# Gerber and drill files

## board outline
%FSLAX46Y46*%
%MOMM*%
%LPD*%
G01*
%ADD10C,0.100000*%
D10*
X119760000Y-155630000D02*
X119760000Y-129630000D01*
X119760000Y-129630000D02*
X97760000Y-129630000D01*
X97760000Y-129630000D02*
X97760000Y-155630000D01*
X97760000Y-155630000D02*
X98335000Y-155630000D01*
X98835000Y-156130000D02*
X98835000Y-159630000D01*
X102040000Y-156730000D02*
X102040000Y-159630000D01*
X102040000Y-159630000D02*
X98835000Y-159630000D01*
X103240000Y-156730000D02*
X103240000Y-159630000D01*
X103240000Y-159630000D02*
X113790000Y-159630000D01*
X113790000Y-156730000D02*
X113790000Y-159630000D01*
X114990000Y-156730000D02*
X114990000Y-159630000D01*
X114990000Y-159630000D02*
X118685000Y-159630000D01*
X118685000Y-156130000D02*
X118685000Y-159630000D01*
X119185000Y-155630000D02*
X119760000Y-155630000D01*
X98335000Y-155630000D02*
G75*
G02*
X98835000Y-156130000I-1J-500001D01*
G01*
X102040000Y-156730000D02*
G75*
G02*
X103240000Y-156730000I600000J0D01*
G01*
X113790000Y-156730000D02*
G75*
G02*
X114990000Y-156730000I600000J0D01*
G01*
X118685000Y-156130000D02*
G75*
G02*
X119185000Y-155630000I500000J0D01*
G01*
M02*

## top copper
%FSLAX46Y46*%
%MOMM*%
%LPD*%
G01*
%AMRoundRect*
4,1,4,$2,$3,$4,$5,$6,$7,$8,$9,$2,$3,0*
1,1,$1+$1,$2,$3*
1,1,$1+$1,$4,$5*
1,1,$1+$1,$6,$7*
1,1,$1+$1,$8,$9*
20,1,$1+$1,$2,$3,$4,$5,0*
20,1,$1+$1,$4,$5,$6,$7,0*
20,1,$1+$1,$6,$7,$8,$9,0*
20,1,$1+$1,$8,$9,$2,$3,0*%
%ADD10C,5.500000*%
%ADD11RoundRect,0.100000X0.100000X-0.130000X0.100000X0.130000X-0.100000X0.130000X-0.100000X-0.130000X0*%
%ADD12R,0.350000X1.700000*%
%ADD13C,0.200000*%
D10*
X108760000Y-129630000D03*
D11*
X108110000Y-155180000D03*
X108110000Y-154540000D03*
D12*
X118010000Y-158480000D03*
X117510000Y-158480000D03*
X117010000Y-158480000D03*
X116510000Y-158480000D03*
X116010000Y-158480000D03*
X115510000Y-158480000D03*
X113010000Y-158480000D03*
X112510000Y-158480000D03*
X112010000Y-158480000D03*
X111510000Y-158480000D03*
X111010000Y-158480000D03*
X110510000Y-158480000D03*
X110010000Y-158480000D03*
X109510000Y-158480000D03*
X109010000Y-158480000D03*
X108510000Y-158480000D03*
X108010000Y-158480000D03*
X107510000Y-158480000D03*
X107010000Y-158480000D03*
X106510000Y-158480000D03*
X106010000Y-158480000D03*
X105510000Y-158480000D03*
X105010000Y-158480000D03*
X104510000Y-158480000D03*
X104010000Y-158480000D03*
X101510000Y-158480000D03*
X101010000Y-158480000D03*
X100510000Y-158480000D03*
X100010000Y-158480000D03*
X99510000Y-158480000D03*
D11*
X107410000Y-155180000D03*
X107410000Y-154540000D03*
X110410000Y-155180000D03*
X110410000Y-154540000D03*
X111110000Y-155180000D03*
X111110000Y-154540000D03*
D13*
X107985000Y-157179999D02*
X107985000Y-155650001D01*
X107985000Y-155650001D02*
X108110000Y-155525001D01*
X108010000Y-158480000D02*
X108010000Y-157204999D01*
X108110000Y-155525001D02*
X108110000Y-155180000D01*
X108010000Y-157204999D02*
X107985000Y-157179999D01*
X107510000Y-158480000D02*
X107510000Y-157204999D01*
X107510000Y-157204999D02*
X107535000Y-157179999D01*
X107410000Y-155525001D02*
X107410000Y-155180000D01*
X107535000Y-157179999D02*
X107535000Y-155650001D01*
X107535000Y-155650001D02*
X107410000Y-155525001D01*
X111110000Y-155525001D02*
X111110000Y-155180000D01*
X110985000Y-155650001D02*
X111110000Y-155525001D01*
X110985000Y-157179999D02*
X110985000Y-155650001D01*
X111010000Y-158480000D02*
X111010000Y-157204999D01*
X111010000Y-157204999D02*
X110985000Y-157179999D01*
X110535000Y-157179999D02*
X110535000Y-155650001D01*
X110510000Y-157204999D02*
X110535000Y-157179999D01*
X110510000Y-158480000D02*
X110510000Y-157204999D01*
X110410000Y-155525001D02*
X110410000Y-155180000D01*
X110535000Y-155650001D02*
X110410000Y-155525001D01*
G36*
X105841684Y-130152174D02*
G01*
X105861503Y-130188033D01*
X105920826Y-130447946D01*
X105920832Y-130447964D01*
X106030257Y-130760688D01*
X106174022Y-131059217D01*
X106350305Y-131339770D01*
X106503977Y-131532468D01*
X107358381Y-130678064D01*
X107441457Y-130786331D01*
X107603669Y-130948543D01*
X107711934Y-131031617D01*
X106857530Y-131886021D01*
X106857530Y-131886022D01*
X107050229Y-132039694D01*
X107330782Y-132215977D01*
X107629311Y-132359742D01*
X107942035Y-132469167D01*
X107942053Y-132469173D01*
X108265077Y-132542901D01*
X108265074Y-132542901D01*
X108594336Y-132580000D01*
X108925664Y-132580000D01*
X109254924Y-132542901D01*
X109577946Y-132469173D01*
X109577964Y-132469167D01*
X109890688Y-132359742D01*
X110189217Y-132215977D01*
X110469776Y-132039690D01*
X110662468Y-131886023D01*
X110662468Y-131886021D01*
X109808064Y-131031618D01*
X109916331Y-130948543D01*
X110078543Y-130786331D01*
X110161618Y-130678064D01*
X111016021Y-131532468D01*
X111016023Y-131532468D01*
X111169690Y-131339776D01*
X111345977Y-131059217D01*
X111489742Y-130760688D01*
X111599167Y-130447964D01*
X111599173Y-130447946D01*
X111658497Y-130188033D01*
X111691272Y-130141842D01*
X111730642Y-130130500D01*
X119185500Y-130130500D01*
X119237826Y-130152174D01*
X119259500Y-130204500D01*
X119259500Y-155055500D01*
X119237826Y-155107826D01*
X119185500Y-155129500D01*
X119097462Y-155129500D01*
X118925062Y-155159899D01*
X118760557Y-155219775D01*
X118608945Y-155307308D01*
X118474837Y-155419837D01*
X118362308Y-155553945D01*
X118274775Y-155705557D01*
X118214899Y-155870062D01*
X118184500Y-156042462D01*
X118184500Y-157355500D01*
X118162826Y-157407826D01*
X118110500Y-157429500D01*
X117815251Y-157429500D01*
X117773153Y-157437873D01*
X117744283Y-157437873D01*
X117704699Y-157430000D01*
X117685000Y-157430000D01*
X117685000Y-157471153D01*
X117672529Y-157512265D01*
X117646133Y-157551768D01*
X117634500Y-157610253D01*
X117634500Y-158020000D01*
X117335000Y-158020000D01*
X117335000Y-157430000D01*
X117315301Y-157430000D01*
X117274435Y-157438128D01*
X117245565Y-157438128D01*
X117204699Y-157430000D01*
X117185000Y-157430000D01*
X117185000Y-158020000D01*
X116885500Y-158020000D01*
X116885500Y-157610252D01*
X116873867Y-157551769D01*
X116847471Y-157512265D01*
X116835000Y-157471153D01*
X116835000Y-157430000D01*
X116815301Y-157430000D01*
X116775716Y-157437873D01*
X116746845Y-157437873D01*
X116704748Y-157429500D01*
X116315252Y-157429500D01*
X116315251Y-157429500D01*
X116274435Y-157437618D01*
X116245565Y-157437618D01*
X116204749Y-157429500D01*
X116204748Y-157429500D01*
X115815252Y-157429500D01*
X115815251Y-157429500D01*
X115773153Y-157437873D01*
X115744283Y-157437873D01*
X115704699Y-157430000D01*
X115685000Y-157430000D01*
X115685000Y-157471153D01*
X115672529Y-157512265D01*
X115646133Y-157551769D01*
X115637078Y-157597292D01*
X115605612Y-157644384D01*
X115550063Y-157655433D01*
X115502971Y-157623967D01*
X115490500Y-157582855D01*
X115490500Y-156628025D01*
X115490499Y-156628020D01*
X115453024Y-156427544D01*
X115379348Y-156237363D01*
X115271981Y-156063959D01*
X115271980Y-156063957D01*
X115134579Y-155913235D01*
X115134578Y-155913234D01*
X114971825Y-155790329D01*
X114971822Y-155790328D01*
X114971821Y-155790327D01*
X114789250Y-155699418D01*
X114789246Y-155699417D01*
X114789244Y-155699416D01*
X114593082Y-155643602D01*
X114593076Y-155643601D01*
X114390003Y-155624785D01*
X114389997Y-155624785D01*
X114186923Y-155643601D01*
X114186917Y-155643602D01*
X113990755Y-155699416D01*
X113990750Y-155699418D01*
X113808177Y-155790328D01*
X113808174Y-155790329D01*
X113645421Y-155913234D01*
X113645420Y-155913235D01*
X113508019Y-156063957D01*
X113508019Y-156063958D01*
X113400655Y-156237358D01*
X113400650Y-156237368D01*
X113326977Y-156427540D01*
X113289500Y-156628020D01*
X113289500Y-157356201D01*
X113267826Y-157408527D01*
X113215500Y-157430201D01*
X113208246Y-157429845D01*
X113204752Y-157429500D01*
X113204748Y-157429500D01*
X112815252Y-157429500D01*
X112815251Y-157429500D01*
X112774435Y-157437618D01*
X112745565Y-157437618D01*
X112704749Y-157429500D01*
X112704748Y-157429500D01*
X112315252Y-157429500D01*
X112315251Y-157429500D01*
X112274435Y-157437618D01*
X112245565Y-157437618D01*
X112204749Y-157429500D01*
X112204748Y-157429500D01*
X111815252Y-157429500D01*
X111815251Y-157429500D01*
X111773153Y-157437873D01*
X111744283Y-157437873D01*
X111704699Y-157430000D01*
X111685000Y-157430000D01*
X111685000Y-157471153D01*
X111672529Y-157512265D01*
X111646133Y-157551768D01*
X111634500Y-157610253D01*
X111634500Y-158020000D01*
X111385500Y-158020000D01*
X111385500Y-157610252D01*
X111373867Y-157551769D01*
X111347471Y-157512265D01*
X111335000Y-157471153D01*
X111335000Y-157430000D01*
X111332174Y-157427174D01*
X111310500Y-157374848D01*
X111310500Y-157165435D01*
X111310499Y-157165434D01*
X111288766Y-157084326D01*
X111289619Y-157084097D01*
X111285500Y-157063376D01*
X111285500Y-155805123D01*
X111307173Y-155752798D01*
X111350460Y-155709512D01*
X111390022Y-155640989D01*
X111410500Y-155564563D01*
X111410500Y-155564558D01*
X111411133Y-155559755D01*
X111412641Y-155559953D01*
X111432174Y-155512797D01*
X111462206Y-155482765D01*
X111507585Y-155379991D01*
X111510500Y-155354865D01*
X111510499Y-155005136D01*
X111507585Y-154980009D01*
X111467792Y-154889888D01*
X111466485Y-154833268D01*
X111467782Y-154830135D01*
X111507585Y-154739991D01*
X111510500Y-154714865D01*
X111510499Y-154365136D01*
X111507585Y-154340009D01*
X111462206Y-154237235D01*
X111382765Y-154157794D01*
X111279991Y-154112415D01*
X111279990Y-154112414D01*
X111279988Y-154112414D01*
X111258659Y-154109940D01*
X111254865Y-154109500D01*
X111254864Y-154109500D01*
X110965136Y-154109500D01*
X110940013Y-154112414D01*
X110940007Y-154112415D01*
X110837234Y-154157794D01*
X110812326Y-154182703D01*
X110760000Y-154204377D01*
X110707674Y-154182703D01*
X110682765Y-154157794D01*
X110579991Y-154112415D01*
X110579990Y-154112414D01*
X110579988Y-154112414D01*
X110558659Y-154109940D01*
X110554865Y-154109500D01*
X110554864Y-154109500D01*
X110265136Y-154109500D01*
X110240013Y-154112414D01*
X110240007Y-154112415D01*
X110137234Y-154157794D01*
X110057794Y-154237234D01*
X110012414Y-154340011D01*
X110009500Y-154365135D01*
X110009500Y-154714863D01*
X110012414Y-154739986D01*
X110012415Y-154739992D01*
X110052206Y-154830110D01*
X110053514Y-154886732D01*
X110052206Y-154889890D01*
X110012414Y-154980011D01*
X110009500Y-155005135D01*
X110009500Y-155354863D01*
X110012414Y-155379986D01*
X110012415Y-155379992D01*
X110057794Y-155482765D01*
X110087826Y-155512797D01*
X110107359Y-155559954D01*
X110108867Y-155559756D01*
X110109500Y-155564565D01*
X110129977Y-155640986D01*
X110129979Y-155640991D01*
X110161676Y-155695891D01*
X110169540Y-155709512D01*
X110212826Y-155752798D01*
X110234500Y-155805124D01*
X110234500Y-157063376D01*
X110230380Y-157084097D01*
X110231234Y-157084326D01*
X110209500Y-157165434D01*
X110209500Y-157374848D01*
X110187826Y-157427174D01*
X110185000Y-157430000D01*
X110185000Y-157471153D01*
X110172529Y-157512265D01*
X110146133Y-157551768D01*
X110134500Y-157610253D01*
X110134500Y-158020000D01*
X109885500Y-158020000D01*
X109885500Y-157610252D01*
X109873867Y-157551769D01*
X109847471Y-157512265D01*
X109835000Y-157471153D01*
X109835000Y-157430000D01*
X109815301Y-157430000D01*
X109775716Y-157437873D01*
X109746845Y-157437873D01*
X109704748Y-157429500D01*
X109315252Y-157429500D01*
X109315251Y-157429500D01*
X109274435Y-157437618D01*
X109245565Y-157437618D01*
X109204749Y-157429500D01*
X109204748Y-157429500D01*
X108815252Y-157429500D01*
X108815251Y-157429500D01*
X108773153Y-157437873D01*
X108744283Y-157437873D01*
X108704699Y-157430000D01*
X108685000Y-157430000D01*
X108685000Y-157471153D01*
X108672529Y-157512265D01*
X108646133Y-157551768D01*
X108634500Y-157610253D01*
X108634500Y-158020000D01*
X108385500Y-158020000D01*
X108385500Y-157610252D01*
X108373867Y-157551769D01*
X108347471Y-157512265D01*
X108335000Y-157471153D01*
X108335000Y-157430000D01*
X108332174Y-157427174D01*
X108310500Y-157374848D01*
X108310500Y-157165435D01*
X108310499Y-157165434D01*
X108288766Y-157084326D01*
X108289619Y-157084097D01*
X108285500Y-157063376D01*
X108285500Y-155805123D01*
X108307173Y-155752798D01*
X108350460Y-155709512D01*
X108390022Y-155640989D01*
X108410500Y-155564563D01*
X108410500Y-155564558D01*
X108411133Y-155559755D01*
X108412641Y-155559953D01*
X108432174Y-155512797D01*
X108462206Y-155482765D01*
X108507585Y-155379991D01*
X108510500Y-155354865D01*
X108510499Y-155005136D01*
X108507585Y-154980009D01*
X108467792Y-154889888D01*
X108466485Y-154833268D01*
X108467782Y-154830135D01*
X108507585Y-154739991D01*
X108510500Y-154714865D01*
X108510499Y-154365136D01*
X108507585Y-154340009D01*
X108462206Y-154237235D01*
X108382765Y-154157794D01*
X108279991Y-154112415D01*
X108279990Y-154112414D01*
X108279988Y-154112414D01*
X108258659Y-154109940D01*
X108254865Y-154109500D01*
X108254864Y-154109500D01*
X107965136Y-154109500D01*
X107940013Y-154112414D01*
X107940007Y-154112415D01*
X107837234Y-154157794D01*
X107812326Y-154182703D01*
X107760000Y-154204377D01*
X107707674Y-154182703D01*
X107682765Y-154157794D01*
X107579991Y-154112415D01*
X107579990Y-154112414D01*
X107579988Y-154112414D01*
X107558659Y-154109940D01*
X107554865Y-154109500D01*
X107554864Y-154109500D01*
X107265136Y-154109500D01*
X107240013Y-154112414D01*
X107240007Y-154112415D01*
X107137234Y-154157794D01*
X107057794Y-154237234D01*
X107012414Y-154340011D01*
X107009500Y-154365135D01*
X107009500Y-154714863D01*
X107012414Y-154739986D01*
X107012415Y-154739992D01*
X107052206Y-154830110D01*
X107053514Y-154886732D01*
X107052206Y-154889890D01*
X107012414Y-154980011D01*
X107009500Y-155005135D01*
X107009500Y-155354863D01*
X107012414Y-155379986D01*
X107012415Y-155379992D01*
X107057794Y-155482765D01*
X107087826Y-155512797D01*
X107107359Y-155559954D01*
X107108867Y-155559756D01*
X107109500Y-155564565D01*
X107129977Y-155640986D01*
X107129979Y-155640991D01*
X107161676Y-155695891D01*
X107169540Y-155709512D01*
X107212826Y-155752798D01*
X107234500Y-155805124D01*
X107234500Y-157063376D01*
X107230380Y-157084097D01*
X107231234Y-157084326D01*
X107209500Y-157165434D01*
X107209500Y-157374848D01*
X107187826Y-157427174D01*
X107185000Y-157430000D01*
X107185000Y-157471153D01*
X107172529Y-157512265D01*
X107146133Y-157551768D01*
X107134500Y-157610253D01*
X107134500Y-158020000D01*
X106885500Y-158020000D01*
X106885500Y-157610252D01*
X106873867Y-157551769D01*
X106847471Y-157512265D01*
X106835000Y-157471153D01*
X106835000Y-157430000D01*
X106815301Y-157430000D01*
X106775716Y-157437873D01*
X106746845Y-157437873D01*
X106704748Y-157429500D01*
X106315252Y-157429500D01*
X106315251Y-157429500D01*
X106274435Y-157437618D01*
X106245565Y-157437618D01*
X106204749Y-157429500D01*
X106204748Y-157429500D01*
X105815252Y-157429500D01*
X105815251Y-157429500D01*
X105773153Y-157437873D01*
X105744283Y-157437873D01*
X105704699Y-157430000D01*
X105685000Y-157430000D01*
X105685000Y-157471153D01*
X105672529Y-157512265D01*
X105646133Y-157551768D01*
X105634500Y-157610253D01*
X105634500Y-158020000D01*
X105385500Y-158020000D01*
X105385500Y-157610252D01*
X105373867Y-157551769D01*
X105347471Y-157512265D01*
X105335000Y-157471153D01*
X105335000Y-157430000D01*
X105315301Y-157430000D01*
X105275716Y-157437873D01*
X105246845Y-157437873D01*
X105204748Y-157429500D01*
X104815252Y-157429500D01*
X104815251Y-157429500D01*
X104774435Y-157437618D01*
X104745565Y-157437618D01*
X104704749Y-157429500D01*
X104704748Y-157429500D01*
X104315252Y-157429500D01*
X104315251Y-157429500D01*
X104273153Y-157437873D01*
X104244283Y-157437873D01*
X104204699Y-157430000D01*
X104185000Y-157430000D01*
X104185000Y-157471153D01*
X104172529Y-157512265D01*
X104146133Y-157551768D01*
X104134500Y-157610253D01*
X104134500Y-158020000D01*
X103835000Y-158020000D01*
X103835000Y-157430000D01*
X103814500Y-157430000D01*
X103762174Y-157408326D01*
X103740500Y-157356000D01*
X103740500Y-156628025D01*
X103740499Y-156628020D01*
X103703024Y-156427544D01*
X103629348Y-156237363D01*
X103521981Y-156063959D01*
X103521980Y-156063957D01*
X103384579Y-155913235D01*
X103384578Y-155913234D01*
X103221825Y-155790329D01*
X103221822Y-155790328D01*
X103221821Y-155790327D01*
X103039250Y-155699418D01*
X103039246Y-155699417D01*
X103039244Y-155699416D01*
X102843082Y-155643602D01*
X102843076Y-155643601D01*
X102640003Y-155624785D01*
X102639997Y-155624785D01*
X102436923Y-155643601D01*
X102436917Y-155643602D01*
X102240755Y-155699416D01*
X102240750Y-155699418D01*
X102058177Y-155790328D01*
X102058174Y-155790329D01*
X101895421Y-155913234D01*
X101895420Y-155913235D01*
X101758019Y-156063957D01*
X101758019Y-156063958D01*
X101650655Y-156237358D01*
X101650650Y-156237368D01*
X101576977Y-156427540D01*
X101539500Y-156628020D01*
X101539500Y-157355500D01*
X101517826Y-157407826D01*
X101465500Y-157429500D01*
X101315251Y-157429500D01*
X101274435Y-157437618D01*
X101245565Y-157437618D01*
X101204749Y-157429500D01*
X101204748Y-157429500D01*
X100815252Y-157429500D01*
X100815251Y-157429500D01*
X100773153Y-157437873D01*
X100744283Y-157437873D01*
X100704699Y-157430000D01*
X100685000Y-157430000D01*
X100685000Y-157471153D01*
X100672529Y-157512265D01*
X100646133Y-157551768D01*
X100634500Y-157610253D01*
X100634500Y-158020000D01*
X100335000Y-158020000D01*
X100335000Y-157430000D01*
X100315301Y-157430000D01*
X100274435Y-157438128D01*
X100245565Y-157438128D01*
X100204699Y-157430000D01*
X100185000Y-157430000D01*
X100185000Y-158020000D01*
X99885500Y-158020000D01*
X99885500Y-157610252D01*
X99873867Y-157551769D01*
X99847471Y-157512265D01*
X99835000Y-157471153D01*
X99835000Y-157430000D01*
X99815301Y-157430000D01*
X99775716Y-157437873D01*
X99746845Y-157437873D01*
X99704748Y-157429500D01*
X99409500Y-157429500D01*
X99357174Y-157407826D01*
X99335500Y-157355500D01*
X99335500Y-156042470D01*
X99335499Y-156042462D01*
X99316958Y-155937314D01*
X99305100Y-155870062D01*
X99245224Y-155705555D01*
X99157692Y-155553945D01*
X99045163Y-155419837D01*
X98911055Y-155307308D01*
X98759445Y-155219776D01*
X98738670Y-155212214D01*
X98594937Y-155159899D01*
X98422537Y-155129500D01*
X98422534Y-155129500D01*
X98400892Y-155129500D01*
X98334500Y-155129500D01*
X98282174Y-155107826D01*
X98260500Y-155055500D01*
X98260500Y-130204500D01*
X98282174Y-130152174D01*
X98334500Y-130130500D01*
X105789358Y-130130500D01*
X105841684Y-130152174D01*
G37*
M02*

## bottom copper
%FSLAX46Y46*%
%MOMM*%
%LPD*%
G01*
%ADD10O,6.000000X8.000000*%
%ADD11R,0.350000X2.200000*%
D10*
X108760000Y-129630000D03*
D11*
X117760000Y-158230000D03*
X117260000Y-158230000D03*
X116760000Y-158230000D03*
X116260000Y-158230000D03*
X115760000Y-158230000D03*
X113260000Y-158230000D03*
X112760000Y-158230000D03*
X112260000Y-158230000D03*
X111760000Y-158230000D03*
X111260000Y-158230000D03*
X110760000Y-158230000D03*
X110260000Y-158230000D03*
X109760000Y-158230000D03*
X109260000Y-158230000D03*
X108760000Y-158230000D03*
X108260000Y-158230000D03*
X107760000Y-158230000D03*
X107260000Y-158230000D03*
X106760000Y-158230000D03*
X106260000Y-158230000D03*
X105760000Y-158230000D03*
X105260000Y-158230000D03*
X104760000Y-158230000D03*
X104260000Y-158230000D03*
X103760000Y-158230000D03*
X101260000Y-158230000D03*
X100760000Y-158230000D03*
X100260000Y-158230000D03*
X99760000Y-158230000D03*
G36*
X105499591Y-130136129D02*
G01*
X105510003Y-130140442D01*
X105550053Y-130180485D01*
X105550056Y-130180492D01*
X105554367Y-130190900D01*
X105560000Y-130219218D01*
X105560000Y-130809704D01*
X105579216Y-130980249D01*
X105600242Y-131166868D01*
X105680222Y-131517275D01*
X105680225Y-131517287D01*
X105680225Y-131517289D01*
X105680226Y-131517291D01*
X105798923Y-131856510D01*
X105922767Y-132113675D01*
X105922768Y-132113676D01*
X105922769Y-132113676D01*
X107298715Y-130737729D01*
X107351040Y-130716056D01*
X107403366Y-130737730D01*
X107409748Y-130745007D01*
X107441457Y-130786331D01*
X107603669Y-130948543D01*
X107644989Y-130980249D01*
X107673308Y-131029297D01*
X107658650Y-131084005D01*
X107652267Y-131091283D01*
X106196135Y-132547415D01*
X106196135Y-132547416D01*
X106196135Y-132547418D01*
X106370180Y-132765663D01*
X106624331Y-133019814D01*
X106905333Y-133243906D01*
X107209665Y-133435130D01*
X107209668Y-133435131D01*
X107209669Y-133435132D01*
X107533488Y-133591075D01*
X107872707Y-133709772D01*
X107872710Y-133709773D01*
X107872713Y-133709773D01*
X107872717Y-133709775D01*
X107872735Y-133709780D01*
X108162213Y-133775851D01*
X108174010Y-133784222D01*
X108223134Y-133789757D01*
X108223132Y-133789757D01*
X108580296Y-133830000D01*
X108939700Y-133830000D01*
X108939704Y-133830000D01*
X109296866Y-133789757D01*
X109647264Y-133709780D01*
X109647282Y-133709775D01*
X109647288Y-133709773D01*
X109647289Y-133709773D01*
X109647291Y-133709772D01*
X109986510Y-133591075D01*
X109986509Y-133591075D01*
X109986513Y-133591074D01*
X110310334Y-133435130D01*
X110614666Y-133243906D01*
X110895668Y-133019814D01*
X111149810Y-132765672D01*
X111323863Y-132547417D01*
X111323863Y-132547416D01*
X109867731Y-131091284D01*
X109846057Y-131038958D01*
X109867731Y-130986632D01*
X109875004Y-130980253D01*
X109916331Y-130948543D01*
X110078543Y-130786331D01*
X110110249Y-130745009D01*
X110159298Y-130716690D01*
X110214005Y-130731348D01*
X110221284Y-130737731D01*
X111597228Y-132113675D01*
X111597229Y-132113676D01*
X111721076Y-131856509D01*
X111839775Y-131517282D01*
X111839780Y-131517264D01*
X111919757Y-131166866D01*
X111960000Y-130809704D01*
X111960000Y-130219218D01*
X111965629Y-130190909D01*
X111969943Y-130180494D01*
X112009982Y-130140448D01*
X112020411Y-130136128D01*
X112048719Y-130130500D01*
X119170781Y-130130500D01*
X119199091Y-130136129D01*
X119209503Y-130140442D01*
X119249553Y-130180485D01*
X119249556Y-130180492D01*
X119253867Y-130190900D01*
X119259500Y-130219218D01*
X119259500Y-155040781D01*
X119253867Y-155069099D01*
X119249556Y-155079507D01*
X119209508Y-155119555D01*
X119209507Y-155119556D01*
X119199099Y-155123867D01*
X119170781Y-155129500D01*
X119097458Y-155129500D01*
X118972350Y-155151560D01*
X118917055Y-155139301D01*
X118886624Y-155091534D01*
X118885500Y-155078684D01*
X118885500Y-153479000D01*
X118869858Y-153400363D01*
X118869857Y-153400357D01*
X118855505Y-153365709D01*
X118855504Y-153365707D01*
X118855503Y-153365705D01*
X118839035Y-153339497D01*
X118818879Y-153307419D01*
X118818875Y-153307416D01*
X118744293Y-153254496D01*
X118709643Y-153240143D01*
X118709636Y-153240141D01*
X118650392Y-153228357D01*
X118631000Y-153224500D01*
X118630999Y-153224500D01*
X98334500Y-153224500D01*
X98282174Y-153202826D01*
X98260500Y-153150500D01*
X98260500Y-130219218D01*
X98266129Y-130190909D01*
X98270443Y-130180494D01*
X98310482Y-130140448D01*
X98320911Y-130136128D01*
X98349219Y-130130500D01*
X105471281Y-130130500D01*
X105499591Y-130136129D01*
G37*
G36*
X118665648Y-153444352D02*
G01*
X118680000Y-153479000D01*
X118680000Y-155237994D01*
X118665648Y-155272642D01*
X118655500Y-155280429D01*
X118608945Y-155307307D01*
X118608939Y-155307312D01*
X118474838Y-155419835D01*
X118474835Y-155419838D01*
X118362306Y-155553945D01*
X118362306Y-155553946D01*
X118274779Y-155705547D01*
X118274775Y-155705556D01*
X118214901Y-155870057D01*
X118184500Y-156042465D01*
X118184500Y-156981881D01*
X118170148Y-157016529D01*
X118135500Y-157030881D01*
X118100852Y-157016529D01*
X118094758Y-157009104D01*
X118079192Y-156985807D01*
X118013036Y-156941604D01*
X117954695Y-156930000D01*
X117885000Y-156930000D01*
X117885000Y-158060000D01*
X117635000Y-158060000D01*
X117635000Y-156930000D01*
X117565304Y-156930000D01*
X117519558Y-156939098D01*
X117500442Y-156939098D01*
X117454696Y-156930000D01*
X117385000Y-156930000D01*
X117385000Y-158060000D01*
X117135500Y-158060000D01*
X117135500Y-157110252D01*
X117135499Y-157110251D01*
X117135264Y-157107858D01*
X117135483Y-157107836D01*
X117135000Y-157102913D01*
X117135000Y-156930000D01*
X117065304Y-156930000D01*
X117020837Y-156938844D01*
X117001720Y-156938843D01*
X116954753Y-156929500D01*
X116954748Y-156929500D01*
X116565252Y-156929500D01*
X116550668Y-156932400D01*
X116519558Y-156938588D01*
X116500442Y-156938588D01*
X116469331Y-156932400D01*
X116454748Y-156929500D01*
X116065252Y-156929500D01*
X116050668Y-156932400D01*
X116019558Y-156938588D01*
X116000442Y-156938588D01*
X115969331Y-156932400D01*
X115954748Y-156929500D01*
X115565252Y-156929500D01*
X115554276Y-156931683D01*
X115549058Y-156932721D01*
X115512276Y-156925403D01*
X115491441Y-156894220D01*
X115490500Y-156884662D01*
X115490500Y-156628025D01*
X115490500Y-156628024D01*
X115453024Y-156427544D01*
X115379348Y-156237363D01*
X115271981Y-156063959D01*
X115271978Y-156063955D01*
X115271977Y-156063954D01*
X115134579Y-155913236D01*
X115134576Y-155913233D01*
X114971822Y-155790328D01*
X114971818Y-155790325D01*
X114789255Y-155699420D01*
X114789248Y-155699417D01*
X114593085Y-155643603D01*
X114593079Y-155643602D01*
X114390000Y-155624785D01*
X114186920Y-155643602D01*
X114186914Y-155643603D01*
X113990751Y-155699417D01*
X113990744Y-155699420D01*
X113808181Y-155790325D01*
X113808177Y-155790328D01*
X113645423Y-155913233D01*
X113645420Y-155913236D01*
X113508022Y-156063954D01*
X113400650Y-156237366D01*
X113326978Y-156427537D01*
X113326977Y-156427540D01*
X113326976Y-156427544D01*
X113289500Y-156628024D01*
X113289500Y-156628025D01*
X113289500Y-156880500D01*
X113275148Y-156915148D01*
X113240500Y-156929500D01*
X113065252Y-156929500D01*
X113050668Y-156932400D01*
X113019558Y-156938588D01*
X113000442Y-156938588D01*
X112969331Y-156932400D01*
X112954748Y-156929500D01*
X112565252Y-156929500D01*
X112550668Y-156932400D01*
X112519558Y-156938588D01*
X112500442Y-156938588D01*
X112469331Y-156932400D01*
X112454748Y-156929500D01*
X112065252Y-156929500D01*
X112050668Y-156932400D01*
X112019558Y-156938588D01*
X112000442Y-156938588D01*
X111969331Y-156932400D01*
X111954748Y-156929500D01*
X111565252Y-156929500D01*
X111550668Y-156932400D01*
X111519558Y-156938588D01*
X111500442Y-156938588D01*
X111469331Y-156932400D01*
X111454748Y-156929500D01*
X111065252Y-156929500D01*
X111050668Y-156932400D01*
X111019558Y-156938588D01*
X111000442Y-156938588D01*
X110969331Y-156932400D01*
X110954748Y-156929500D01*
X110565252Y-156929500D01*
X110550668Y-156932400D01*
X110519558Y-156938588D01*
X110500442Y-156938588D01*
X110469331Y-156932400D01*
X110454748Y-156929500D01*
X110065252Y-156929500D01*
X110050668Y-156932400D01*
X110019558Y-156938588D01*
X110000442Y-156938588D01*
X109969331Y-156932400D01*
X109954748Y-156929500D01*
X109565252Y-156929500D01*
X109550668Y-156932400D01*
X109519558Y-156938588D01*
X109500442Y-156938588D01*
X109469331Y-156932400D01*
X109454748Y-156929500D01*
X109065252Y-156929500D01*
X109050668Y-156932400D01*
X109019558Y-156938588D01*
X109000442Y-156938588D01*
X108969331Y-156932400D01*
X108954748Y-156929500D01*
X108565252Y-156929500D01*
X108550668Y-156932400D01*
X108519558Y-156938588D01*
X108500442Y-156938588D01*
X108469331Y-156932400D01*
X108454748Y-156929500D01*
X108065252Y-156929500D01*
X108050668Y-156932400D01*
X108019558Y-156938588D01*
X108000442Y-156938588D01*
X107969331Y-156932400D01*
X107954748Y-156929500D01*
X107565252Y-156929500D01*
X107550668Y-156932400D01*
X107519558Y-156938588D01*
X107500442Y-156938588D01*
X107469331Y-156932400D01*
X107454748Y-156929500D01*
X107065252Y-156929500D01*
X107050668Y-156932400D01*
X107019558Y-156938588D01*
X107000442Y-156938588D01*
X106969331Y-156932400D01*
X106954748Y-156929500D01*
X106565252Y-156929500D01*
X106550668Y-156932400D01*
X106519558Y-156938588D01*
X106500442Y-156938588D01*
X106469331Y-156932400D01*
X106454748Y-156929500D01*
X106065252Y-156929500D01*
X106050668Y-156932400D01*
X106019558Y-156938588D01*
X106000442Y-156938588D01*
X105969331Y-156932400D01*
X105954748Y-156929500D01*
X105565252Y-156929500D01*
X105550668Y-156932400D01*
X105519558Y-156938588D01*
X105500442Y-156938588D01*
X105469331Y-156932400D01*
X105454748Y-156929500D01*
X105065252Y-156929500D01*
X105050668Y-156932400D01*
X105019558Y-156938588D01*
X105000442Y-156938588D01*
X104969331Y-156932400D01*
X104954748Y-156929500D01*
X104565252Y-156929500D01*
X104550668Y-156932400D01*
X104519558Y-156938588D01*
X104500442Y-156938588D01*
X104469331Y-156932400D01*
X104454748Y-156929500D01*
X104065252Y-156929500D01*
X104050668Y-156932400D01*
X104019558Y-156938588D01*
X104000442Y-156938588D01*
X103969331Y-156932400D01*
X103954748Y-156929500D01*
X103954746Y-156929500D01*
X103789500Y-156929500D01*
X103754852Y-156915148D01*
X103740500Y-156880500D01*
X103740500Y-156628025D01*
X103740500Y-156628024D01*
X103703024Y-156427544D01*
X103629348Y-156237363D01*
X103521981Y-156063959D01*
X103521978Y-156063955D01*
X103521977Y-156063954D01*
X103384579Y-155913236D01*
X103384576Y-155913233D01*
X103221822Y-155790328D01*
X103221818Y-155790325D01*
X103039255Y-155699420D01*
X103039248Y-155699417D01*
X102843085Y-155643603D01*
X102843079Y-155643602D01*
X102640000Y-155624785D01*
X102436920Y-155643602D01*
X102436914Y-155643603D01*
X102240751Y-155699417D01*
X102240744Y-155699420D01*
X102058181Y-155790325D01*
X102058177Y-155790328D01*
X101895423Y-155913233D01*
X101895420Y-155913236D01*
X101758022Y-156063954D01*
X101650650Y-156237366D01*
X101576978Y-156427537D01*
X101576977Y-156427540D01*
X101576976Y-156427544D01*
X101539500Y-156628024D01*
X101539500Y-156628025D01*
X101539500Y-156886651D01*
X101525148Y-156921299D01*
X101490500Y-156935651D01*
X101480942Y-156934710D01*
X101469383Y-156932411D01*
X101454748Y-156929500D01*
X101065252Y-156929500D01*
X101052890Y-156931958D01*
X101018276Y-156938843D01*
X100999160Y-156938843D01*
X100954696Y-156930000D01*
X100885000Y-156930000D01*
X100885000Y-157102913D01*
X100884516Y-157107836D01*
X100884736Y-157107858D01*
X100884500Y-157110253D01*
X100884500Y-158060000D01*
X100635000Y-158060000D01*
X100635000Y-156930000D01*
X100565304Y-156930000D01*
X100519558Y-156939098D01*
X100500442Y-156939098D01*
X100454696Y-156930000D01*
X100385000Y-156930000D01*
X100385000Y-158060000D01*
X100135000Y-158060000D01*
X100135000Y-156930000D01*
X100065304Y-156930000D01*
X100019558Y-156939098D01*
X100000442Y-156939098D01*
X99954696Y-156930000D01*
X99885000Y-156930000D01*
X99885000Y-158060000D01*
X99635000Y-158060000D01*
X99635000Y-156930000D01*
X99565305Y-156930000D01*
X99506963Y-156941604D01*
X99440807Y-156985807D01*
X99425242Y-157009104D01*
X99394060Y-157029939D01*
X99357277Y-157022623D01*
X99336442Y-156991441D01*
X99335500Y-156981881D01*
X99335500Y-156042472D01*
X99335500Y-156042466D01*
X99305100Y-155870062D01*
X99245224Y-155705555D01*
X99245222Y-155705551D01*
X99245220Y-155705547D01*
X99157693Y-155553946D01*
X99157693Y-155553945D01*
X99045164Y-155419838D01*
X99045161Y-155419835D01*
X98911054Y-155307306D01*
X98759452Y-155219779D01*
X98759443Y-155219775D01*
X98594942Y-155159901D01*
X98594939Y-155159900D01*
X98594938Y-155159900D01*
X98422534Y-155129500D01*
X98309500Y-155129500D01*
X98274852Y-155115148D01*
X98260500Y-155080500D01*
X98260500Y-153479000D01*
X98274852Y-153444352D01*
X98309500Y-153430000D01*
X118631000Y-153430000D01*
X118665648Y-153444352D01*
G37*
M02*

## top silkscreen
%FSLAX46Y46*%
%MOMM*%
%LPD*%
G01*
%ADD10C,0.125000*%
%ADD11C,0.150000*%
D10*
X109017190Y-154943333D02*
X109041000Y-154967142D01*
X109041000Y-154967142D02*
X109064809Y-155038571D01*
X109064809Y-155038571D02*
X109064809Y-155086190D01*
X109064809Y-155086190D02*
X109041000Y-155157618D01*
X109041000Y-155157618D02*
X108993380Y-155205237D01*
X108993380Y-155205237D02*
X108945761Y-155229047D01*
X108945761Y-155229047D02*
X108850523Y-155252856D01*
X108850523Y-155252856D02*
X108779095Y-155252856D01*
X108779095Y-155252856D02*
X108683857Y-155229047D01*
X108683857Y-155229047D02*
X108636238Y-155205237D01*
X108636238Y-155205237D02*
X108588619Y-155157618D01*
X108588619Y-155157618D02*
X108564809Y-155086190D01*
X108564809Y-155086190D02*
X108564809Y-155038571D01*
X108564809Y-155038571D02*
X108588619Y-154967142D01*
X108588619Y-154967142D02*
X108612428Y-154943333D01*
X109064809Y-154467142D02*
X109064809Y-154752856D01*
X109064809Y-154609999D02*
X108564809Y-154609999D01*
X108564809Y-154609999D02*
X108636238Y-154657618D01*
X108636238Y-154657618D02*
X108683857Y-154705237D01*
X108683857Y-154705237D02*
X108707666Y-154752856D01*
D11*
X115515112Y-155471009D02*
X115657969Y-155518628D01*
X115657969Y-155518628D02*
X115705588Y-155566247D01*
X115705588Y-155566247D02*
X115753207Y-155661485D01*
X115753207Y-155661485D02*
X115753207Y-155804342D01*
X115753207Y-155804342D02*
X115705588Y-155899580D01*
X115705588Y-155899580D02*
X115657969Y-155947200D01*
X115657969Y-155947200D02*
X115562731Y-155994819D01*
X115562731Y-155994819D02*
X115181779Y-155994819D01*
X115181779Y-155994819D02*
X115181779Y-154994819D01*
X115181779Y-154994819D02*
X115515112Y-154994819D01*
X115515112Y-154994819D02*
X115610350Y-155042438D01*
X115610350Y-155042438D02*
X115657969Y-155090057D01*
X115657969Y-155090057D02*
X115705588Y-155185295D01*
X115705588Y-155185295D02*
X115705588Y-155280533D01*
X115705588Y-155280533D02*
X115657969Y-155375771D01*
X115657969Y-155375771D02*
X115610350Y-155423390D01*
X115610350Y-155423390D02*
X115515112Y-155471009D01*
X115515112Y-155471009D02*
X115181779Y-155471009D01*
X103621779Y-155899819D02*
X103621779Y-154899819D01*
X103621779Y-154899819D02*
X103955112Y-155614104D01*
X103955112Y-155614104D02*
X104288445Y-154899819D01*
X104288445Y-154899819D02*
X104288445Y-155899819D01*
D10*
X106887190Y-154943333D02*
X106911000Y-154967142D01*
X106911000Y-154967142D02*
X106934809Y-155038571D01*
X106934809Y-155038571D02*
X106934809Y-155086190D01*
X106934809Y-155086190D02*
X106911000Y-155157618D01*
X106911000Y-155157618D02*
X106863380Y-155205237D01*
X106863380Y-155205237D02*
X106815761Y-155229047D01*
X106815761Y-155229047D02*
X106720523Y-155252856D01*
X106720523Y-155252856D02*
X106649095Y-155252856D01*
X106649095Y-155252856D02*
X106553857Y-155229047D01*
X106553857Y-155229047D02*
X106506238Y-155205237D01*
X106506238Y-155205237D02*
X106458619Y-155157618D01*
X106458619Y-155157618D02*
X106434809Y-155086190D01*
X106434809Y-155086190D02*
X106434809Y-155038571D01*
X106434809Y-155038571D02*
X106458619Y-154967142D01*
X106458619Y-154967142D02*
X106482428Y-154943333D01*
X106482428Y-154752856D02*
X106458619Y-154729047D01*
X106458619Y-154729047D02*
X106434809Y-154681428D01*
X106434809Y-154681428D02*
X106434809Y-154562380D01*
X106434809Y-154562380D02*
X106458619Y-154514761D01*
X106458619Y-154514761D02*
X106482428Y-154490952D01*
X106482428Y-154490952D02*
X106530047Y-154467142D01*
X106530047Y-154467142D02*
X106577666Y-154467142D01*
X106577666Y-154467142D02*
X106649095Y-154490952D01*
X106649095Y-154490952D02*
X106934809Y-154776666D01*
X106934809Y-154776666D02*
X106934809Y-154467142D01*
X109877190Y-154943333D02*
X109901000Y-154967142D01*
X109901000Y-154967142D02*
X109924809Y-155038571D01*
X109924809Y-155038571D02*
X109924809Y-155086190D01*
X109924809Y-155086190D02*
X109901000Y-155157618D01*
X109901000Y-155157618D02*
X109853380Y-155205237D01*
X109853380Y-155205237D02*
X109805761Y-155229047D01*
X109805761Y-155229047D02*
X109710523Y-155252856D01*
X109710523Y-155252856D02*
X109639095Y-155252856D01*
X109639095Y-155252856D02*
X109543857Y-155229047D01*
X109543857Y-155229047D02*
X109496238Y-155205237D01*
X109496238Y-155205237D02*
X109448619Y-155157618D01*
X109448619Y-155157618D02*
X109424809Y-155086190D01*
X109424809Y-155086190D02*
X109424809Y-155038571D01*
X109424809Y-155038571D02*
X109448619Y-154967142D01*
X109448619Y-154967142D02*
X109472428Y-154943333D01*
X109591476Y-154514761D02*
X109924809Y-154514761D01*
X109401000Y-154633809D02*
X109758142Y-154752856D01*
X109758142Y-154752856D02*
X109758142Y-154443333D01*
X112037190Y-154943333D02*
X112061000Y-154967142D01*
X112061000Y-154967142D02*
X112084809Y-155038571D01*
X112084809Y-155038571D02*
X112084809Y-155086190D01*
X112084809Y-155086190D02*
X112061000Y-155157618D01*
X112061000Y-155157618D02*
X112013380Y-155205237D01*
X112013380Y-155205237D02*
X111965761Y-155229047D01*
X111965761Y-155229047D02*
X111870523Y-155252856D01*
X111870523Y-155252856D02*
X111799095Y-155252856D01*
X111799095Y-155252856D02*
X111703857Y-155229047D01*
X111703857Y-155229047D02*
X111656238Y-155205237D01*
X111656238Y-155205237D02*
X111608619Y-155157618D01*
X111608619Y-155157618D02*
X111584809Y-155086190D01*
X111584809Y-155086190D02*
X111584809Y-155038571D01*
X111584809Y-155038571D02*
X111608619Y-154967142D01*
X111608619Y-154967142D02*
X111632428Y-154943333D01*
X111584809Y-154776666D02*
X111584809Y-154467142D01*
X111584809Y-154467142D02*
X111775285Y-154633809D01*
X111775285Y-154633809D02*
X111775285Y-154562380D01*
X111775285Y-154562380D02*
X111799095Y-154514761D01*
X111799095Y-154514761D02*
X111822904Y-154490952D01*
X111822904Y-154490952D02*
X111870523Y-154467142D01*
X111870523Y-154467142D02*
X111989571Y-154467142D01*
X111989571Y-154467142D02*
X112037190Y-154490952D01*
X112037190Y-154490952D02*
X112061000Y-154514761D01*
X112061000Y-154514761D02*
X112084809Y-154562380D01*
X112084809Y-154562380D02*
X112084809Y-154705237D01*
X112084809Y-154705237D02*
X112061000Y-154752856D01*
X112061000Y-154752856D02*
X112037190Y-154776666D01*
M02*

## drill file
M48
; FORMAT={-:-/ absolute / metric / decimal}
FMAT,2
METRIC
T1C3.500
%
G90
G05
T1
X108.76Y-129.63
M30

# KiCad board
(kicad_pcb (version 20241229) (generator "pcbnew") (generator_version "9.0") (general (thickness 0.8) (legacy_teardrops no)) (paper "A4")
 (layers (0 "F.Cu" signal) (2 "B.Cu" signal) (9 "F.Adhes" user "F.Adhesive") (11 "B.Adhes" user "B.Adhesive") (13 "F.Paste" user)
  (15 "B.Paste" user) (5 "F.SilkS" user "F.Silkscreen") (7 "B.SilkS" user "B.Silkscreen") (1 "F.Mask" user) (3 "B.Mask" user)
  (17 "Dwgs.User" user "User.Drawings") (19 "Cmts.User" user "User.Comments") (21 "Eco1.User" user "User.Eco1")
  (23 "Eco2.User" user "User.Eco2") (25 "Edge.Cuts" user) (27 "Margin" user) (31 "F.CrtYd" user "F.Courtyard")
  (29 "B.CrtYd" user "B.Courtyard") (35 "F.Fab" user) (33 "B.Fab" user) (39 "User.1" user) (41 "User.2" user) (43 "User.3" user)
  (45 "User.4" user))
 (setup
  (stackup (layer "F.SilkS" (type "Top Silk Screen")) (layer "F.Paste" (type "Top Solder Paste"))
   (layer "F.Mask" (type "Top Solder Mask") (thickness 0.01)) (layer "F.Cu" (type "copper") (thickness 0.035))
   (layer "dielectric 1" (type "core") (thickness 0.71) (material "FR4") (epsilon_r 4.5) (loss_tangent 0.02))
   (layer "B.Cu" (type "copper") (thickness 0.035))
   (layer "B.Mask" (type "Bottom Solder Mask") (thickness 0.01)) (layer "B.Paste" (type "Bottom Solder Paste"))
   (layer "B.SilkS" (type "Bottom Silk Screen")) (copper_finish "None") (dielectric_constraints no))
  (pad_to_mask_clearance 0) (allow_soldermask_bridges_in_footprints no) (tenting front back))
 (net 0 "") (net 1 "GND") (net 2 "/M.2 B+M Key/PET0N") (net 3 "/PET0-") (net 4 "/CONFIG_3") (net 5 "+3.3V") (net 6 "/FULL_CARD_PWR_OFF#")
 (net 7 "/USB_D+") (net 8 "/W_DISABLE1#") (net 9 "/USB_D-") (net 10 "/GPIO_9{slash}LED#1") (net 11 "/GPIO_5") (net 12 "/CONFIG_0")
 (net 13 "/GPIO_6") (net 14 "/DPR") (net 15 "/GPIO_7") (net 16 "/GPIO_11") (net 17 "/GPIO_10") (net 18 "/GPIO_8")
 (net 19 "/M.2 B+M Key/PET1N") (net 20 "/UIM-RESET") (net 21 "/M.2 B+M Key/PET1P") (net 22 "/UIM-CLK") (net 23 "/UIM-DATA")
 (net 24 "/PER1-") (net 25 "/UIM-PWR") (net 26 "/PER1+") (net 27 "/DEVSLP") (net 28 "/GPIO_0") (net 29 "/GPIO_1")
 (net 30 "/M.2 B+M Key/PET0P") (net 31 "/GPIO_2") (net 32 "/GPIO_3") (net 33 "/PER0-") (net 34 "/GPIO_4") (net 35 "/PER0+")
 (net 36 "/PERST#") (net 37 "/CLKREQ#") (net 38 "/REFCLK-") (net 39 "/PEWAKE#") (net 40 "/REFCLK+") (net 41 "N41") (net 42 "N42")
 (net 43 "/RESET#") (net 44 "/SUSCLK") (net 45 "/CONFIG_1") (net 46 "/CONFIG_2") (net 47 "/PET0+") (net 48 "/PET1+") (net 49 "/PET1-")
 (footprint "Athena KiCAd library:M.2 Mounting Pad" (layer "F.Cu") (at 108.76 129.63)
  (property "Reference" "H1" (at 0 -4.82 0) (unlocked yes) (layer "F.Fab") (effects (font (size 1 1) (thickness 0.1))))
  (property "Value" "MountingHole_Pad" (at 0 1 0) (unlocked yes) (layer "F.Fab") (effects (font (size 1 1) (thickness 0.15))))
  (pad "1" thru_hole circle (at 0 0) (size 5.5 5.5) (drill 3.5) (layers "*.Cu" "*.Mask") (remove_unused_layers no) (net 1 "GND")
   (padstack (mode front_inner_back)
    (layer "Inner" (shape circle) (size 5.5 5.5) (zone_connect -1))
    (layer "B.Cu" (shape oval) (size 6 8) (thermal_bridge_angle 45) (zone_connect -1)))))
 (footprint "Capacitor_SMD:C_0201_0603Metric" (layer "F.Cu") (at 108.11 154.86 90)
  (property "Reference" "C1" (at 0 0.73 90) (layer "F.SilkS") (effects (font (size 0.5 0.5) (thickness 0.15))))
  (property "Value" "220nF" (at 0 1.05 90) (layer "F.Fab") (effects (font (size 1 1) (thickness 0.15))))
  (pad "" smd roundrect (at -0.345 0 90) (size 0.318 0.36) (layers "F.Paste") (roundrect_rratio 0.25))
  (pad "" smd roundrect (at 0.345 0 90) (size 0.318 0.36) (layers "F.Paste") (roundrect_rratio 0.25))
  (pad "1" smd roundrect (at -0.32 0 90) (size 0.46 0.4) (layers "F.Cu" "F.Mask") (roundrect_rratio 0.25) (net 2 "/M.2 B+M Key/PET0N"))
  (pad "2" smd roundrect (at 0.32 0 90) (size 0.46 0.4) (layers "F.Cu" "F.Mask") (roundrect_rratio 0.25) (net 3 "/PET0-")))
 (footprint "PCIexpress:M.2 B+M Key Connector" (layer "F.Cu") (at 108.76 158.52)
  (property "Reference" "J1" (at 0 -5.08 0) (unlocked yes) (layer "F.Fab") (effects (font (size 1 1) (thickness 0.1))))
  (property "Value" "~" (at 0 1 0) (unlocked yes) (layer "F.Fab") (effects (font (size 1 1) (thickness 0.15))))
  (fp_line (start -11 -2.89) (end -10.425 -2.89) (stroke (width 0.1) (type default)) (layer "Edge.Cuts"))
  (fp_line (start -9.925 -2.39) (end -9.925 1.11) (stroke (width 0.1) (type default)) (layer "Edge.Cuts"))
  (fp_line (start -6.72 -1.79) (end -6.72 1.11) (stroke (width 0.1) (type default)) (layer "Edge.Cuts"))
  (fp_line (start -6.72 1.11) (end -9.925 1.11) (stroke (width 0.1) (type default)) (layer "Edge.Cuts"))
  (fp_line (start -5.52 -1.79) (end -5.52 1.11) (stroke (width 0.1) (type default)) (layer "Edge.Cuts"))
  (fp_line (start -5.52 1.11) (end 5.03 1.11) (stroke (width 0.1) (type default)) (layer "Edge.Cuts"))
  (fp_line (start 5.03 -1.79) (end 5.03 1.11) (stroke (width 0.1) (type default)) (layer "Edge.Cuts"))
  (fp_line (start 6.23 -1.79) (end 6.23 1.11) (stroke (width 0.1) (type default)) (layer "Edge.Cuts"))
  (fp_line (start 6.23 1.11) (end 9.925 1.11) (stroke (width 0.1) (type default)) (layer "Edge.Cuts"))
  (fp_line (start 9.925 -2.39) (end 9.925 1.11) (stroke (width 0.1) (type default)) (layer "Edge.Cuts"))
  (fp_line (start 10.425 -2.89) (end 11 -2.89) (stroke (width 0.1) (type default)) (layer "Edge.Cuts"))
  (fp_arc (start -10.425 -2.89) (mid -10.071447 -2.743553) (end -9.925 -2.39) (stroke (width 0.1) (type default)) (layer "Edge.Cuts"))
  (fp_arc (start -6.72 -1.79) (mid -6.12 -2.39) (end -5.52 -1.79) (stroke (width 0.1) (type default)) (layer "Edge.Cuts"))
  (fp_arc (start 5.03 -1.79) (mid 5.63 -2.39) (end 6.23 -1.79) (stroke (width 0.1) (type default)) (layer "Edge.Cuts"))
  (fp_arc (start 9.925 -2.39) (mid 10.071447 -2.743553) (end 10.425 -2.89) (stroke (width 0.1) (type default)) (layer "Edge.Cuts"))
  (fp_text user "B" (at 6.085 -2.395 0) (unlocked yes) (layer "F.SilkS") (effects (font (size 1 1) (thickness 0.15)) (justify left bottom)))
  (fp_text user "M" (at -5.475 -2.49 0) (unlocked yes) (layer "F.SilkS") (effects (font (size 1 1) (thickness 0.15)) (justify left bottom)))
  (pad "1" smd rect (at 9.25 -0.04 180) (size 0.35 1.7) (layers "F.Cu") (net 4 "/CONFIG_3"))
  (pad "2" smd rect (at 9 -0.29 180) (size 0.35 2.2) (layers "B.Cu") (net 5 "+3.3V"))
  (pad "3" smd rect (at 8.75 -0.04 180) (size 0.35 1.7) (layers "F.Cu") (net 1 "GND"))
  (pad "4" smd rect (at 8.5 -0.29 180) (size 0.35 2.2) (layers "B.Cu") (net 5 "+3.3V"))
  (pad "5" smd rect (at 8.25 -0.04 180) (size 0.35 1.7) (layers "F.Cu") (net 1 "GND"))
  (pad "6" smd rect (at 8 -0.29 180) (size 0.35 2.2) (layers "B.Cu") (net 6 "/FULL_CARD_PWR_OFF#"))
  (pad "7" smd rect (at 7.75 -0.04 180) (size 0.35 1.7) (layers "F.Cu") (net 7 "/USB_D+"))
  (pad "8" smd rect (at 7.5 -0.29 180) (size 0.35 2.2) (layers "B.Cu") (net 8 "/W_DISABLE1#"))
  (pad "9" smd rect (at 7.25 -0.04 180) (size 0.35 1.7) (layers "F.Cu") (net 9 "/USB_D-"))
  (pad "10" smd rect (at 7 -0.29 180) (size 0.35 2.2) (layers "B.Cu") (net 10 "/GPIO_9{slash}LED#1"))
  (pad "11" smd rect (at 6.75 -0.04 180) (size 0.35 1.7) (layers "F.Cu") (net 1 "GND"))
  (pad "20" smd rect (at 4.5 -0.29 180) (size 0.35 2.2) (layers "B.Cu") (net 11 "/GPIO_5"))
  (pad "21" smd rect (at 4.25 -0.04 180) (size 0.35 1.7) (layers "F.Cu") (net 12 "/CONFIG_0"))
  (pad "22" smd rect (at 4 -0.29 180) (size 0.35 2.2) (layers "B.Cu") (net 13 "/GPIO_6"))
  (pad "23" smd rect (at 3.75 -0.04 180) (size 0.35 1.7) (layers "F.Cu") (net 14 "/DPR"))
  (pad "24" smd rect (at 3.5 -0.29 180) (size 0.35 2.2) (layers "B.Cu") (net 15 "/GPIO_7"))
  (pad "25" smd rect (at 3.25 -0.04 180) (size 0.35 1.7) (layers "F.Cu") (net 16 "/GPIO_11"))
  (pad "26" smd rect (at 3 -0.29 180) (size 0.35 2.2) (layers "B.Cu") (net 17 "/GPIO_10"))
  (pad "27" smd rect (at 2.75 -0.04 180) (size 0.35 1.7) (layers "F.Cu") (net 1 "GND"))
  (pad "28" smd rect (at 2.5 -0.29 180) (size 0.35 2.2) (layers "B.Cu") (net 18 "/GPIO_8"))
  (pad "29" smd rect (at 2.25 -0.04 180) (size 0.35 1.7) (layers "F.Cu") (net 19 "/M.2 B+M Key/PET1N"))
  (pad "30" smd rect (at 2 -0.29 180) (size 0.35 2.2) (layers "B.Cu") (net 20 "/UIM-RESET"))
  (pad "31" smd rect (at 1.75 -0.04 180) (size 0.35 1.7) (layers "F.Cu") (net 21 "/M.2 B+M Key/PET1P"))
  (pad "32" smd rect (at 1.5 -0.29 180) (size 0.35 2.2) (layers "B.Cu") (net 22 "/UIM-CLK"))
  (pad "33" smd rect (at 1.25 -0.04 180) (size 0.35 1.7) (layers "F.Cu") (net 1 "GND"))
  (pad "34" smd rect (at 1 -0.29 180) (size 0.35 2.2) (layers "B.Cu") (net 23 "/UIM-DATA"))
  (pad "35" smd rect (at 0.75 -0.04 180) (size 0.35 1.7) (layers "F.Cu") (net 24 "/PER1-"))
  (pad "36" smd rect (at 0.5 -0.29 180) (size 0.35 2.2) (layers "B.Cu") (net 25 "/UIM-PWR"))
  (pad "37" smd rect (at 0.25 -0.04 180) (size 0.35 1.7) (layers "F.Cu") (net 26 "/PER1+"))
  (pad "38" smd rect (at 0 -0.29 180) (size 0.35 2.2) (layers "B.Cu") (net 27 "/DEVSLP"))
  (pad "39" smd rect (at -0.25 -0.04 180) (size 0.35 1.7) (layers "F.Cu") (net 1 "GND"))
  (pad "40" smd rect (at -0.5 -0.29 180) (size 0.35 2.2) (layers "B.Cu") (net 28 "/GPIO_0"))
  (pad "41" smd rect (at -0.75 -0.04 180) (size 0.35 1.7) (layers "F.Cu") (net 2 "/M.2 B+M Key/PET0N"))
  (pad "42" smd rect (at -1 -0.29 180) (size 0.35 2.2) (layers "B.Cu") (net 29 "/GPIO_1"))
  (pad "43" smd rect (at -1.25 -0.04 180) (size 0.35 1.7) (layers "F.Cu") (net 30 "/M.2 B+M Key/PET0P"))
  (pad "44" smd rect (at -1.5 -0.29 180) (size 0.35 2.2) (layers "B.Cu") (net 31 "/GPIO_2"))
  (pad "45" smd rect (at -1.75 -0.04 180) (size 0.35 1.7) (layers "F.Cu") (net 1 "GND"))
  (pad "46" smd rect (at -2 -0.29 180) (size 0.35 2.2) (layers "B.Cu") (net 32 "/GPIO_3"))
  (pad "47" smd rect (at -2.25 -0.04 180) (size 0.35 1.7) (layers "F.Cu") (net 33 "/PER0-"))
  (pad "48" smd rect (at -2.5 -0.29 180) (size 0.35 2.2) (layers "B.Cu") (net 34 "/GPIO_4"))
  (pad "49" smd rect (at -2.75 -0.04 180) (size 0.35 1.7) (layers "F.Cu") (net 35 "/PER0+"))
  (pad "50" smd rect (at -3 -0.29 180) (size 0.35 2.2) (layers "B.Cu") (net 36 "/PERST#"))
  (pad "51" smd rect (at -3.25 -0.04 180) (size 0.35 1.7) (layers "F.Cu") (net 1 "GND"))
  (pad "52" smd rect (at -3.5 -0.29 180) (size 0.35 2.2) (layers "B.Cu") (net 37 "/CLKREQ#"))
  (pad "53" smd rect (at -3.75 -0.04 180) (size 0.35 1.7) (layers "F.Cu") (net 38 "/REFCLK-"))
  (pad "54" smd rect (at -4 -0.29 180) (size 0.35 2.2) (layers "B.Cu") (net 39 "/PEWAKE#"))
  (pad "55" smd rect (at -4.25 -0.04 180) (size 0.35 1.7) (layers "F.Cu") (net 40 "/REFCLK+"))
  (pad "56" smd rect (at -4.5 -0.29 180) (size 0.35 2.2) (layers "B.Cu") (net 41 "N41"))
  (pad "57" smd rect (at -4.75 -0.04 180) (size 0.35 1.7) (layers "F.Cu") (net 1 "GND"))
  (pad "58" smd rect (at -5 -0.29 180) (size 0.35 2.2) (layers "B.Cu") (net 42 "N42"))
  (pad "67" smd rect (at -7.25 -0.04 180) (size 0.35 1.7) (layers "F.Cu") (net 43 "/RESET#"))
  (pad "68" smd rect (at -7.5 -0.29 180) (size 0.35 2.2) (layers "B.Cu") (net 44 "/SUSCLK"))
  (pad "69" smd rect (at -7.75 -0.04 180) (size 0.35 1.7) (layers "F.Cu") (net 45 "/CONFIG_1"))
  (pad "70" smd rect (at -8 -0.29 180) (size 0.35 2.2) (layers "B.Cu") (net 5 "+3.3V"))
  (pad "71" smd rect (at -8.25 -0.04 180) (size 0.35 1.7) (layers "F.Cu") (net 1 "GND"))
  (pad "72" smd rect (at -8.5 -0.29 180) (size 0.35 2.2) (layers "B.Cu") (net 5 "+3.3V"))
  (pad "73" smd rect (at -8.75 -0.04 180) (size 0.35 1.7) (layers "F.Cu") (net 1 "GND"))
  (pad "74" smd rect (at -9 -0.29 180) (size 0.35 2.2) (layers "B.Cu") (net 5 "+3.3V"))
  (pad "75" smd rect (at -9.25 -0.04 180) (size 0.35 1.7) (layers "F.Cu") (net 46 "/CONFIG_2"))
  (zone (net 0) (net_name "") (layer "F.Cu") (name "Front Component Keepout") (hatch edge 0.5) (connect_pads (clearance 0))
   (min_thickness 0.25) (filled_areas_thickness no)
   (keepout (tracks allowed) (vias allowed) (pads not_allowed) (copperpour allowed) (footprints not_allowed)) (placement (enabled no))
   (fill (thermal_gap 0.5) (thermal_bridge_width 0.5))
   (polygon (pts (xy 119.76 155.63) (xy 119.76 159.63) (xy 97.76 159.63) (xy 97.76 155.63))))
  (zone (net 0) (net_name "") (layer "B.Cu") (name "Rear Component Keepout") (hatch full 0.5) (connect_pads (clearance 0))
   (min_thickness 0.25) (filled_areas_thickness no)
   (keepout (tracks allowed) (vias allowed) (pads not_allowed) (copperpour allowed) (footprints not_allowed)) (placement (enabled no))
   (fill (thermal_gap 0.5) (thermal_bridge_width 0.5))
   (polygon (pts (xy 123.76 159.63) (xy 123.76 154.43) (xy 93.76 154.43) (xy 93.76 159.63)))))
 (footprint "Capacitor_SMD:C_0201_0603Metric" (layer "F.Cu") (at 107.41 154.86 90)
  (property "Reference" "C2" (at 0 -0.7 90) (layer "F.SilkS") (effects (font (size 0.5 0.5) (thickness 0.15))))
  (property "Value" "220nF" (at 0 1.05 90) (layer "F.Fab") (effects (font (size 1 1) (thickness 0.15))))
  (pad "" smd roundrect (at -0.345 0 90) (size 0.318 0.36) (layers "F.Paste") (roundrect_rratio 0.25))
  (pad "" smd roundrect (at 0.345 0 90) (size 0.318 0.36) (layers "F.Paste") (roundrect_rratio 0.25))
  (pad "1" smd roundrect (at -0.32 0 90) (size 0.46 0.4) (layers "F.Cu" "F.Mask") (roundrect_rratio 0.25) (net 30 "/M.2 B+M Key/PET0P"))
  (pad "2" smd roundrect (at 0.32 0 90) (size 0.46 0.4) (layers "F.Cu" "F.Mask") (roundrect_rratio 0.25) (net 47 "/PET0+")))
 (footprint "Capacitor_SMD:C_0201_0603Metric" (layer "F.Cu") (at 110.41 154.86 90)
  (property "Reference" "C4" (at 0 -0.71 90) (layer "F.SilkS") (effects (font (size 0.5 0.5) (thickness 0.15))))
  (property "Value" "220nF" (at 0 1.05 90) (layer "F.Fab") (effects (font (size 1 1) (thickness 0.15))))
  (pad "" smd roundrect (at -0.345 0 90) (size 0.318 0.36) (layers "F.Paste") (roundrect_rratio 0.25))
  (pad "" smd roundrect (at 0.345 0 90) (size 0.318 0.36) (layers "F.Paste") (roundrect_rratio 0.25))
  (pad "1" smd roundrect (at -0.32 0 90) (size 0.46 0.4) (layers "F.Cu" "F.Mask") (roundrect_rratio 0.25) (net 21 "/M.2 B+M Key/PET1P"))
  (pad "2" smd roundrect (at 0.32 0 90) (size 0.46 0.4) (layers "F.Cu" "F.Mask") (roundrect_rratio 0.25) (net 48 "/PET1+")))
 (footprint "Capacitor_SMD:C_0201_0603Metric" (layer "F.Cu") (at 111.11 154.86 90)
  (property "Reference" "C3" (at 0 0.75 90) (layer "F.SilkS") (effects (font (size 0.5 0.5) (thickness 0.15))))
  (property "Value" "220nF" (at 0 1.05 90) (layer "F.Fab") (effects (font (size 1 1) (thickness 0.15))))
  (pad "" smd roundrect (at -0.345 0 90) (size 0.318 0.36) (layers "F.Paste") (roundrect_rratio 0.25))
  (pad "" smd roundrect (at 0.345 0 90) (size 0.318 0.36) (layers "F.Paste") (roundrect_rratio 0.25))
  (pad "1" smd roundrect (at -0.32 0 90) (size 0.46 0.4) (layers "F.Cu" "F.Mask") (roundrect_rratio 0.25) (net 19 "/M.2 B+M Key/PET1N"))
  (pad "2" smd roundrect (at 0.32 0 90) (size 0.46 0.4) (layers "F.Cu" "F.Mask") (roundrect_rratio 0.25) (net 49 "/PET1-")))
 (gr_line (start 119.76 155.63) (end 119.76 129.63) (stroke (width 0.1) (type default)) (layer "Edge.Cuts"))
 (gr_line (start 119.76 129.63) (end 97.76 129.63) (stroke (width 0.1) (type default)) (layer "Edge.Cuts"))
 (gr_line (start 97.76 129.63) (end 97.76 155.63) (stroke (width 0.1) (type default)) (layer "Edge.Cuts"))
 (segment (start 107.985 157.179999) (end 107.985 155.650001) (width 0.2) (layer "F.Cu") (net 2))
 (segment (start 107.985 155.650001) (end 108.11 155.525001) (width 0.2) (layer "F.Cu") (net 2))
 (segment (start 108.01 158.48) (end 108.01 157.204999) (width 0.2) (layer "F.Cu") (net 2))
 (segment (start 108.11 155.525001) (end 108.11 155.18) (width 0.2) (layer "F.Cu") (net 2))
 (segment (start 108.01 157.204999) (end 107.985 157.179999) (width 0.2) (layer "F.Cu") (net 2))
 (segment (start 107.51 158.48) (end 107.51 157.204999) (width 0.2) (layer "F.Cu") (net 30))
 (segment (start 107.51 157.204999) (end 107.535 157.179999) (width 0.2) (layer "F.Cu") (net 30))
 (segment (start 107.41 155.525001) (end 107.41 155.18) (width 0.2) (layer "F.Cu") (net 30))
 (segment (start 107.535 157.179999) (end 107.535 155.650001) (width 0.2) (layer "F.Cu") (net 30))
 (segment (start 107.535 155.650001) (end 107.41 155.525001) (width 0.2) (layer "F.Cu") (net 30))
 (segment (start 111.11 155.525001) (end 111.11 155.18) (width 0.2) (layer "F.Cu") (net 19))
 (segment (start 110.985 155.650001) (end 111.11 155.525001) (width 0.2) (layer "F.Cu") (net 19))
 (segment (start 110.985 157.179999) (end 110.985 155.650001) (width 0.2) (layer "F.Cu") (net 19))
 (segment (start 111.01 158.48) (end 111.01 157.204999) (width 0.2) (layer "F.Cu") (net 19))
 (segment (start 111.01 157.204999) (end 110.985 157.179999) (width 0.2) (layer "F.Cu") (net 19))
 (segment (start 110.535 157.179999) (end 110.535 155.650001) (width 0.2) (layer "F.Cu") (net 21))
 (segment (start 110.51 157.204999) (end 110.535 157.179999) (width 0.2) (layer "F.Cu") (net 21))
 (segment (start 110.51 158.48) (end 110.51 157.204999) (width 0.2) (layer "F.Cu") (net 21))
 (segment (start 110.41 155.525001) (end 110.41 155.18) (width 0.2) (layer "F.Cu") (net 21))
 (segment (start 110.535 155.650001) (end 110.41 155.525001) (width 0.2) (layer "F.Cu") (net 21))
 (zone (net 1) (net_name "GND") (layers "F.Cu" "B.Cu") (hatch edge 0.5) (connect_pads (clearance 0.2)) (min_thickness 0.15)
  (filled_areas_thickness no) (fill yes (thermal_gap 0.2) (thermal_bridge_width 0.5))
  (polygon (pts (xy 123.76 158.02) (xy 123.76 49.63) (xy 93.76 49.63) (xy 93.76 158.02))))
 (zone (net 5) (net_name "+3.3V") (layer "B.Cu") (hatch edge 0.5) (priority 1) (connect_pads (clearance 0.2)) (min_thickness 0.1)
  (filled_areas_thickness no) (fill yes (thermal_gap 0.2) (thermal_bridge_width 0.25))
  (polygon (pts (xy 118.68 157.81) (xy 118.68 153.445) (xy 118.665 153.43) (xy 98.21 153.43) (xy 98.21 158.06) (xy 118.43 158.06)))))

